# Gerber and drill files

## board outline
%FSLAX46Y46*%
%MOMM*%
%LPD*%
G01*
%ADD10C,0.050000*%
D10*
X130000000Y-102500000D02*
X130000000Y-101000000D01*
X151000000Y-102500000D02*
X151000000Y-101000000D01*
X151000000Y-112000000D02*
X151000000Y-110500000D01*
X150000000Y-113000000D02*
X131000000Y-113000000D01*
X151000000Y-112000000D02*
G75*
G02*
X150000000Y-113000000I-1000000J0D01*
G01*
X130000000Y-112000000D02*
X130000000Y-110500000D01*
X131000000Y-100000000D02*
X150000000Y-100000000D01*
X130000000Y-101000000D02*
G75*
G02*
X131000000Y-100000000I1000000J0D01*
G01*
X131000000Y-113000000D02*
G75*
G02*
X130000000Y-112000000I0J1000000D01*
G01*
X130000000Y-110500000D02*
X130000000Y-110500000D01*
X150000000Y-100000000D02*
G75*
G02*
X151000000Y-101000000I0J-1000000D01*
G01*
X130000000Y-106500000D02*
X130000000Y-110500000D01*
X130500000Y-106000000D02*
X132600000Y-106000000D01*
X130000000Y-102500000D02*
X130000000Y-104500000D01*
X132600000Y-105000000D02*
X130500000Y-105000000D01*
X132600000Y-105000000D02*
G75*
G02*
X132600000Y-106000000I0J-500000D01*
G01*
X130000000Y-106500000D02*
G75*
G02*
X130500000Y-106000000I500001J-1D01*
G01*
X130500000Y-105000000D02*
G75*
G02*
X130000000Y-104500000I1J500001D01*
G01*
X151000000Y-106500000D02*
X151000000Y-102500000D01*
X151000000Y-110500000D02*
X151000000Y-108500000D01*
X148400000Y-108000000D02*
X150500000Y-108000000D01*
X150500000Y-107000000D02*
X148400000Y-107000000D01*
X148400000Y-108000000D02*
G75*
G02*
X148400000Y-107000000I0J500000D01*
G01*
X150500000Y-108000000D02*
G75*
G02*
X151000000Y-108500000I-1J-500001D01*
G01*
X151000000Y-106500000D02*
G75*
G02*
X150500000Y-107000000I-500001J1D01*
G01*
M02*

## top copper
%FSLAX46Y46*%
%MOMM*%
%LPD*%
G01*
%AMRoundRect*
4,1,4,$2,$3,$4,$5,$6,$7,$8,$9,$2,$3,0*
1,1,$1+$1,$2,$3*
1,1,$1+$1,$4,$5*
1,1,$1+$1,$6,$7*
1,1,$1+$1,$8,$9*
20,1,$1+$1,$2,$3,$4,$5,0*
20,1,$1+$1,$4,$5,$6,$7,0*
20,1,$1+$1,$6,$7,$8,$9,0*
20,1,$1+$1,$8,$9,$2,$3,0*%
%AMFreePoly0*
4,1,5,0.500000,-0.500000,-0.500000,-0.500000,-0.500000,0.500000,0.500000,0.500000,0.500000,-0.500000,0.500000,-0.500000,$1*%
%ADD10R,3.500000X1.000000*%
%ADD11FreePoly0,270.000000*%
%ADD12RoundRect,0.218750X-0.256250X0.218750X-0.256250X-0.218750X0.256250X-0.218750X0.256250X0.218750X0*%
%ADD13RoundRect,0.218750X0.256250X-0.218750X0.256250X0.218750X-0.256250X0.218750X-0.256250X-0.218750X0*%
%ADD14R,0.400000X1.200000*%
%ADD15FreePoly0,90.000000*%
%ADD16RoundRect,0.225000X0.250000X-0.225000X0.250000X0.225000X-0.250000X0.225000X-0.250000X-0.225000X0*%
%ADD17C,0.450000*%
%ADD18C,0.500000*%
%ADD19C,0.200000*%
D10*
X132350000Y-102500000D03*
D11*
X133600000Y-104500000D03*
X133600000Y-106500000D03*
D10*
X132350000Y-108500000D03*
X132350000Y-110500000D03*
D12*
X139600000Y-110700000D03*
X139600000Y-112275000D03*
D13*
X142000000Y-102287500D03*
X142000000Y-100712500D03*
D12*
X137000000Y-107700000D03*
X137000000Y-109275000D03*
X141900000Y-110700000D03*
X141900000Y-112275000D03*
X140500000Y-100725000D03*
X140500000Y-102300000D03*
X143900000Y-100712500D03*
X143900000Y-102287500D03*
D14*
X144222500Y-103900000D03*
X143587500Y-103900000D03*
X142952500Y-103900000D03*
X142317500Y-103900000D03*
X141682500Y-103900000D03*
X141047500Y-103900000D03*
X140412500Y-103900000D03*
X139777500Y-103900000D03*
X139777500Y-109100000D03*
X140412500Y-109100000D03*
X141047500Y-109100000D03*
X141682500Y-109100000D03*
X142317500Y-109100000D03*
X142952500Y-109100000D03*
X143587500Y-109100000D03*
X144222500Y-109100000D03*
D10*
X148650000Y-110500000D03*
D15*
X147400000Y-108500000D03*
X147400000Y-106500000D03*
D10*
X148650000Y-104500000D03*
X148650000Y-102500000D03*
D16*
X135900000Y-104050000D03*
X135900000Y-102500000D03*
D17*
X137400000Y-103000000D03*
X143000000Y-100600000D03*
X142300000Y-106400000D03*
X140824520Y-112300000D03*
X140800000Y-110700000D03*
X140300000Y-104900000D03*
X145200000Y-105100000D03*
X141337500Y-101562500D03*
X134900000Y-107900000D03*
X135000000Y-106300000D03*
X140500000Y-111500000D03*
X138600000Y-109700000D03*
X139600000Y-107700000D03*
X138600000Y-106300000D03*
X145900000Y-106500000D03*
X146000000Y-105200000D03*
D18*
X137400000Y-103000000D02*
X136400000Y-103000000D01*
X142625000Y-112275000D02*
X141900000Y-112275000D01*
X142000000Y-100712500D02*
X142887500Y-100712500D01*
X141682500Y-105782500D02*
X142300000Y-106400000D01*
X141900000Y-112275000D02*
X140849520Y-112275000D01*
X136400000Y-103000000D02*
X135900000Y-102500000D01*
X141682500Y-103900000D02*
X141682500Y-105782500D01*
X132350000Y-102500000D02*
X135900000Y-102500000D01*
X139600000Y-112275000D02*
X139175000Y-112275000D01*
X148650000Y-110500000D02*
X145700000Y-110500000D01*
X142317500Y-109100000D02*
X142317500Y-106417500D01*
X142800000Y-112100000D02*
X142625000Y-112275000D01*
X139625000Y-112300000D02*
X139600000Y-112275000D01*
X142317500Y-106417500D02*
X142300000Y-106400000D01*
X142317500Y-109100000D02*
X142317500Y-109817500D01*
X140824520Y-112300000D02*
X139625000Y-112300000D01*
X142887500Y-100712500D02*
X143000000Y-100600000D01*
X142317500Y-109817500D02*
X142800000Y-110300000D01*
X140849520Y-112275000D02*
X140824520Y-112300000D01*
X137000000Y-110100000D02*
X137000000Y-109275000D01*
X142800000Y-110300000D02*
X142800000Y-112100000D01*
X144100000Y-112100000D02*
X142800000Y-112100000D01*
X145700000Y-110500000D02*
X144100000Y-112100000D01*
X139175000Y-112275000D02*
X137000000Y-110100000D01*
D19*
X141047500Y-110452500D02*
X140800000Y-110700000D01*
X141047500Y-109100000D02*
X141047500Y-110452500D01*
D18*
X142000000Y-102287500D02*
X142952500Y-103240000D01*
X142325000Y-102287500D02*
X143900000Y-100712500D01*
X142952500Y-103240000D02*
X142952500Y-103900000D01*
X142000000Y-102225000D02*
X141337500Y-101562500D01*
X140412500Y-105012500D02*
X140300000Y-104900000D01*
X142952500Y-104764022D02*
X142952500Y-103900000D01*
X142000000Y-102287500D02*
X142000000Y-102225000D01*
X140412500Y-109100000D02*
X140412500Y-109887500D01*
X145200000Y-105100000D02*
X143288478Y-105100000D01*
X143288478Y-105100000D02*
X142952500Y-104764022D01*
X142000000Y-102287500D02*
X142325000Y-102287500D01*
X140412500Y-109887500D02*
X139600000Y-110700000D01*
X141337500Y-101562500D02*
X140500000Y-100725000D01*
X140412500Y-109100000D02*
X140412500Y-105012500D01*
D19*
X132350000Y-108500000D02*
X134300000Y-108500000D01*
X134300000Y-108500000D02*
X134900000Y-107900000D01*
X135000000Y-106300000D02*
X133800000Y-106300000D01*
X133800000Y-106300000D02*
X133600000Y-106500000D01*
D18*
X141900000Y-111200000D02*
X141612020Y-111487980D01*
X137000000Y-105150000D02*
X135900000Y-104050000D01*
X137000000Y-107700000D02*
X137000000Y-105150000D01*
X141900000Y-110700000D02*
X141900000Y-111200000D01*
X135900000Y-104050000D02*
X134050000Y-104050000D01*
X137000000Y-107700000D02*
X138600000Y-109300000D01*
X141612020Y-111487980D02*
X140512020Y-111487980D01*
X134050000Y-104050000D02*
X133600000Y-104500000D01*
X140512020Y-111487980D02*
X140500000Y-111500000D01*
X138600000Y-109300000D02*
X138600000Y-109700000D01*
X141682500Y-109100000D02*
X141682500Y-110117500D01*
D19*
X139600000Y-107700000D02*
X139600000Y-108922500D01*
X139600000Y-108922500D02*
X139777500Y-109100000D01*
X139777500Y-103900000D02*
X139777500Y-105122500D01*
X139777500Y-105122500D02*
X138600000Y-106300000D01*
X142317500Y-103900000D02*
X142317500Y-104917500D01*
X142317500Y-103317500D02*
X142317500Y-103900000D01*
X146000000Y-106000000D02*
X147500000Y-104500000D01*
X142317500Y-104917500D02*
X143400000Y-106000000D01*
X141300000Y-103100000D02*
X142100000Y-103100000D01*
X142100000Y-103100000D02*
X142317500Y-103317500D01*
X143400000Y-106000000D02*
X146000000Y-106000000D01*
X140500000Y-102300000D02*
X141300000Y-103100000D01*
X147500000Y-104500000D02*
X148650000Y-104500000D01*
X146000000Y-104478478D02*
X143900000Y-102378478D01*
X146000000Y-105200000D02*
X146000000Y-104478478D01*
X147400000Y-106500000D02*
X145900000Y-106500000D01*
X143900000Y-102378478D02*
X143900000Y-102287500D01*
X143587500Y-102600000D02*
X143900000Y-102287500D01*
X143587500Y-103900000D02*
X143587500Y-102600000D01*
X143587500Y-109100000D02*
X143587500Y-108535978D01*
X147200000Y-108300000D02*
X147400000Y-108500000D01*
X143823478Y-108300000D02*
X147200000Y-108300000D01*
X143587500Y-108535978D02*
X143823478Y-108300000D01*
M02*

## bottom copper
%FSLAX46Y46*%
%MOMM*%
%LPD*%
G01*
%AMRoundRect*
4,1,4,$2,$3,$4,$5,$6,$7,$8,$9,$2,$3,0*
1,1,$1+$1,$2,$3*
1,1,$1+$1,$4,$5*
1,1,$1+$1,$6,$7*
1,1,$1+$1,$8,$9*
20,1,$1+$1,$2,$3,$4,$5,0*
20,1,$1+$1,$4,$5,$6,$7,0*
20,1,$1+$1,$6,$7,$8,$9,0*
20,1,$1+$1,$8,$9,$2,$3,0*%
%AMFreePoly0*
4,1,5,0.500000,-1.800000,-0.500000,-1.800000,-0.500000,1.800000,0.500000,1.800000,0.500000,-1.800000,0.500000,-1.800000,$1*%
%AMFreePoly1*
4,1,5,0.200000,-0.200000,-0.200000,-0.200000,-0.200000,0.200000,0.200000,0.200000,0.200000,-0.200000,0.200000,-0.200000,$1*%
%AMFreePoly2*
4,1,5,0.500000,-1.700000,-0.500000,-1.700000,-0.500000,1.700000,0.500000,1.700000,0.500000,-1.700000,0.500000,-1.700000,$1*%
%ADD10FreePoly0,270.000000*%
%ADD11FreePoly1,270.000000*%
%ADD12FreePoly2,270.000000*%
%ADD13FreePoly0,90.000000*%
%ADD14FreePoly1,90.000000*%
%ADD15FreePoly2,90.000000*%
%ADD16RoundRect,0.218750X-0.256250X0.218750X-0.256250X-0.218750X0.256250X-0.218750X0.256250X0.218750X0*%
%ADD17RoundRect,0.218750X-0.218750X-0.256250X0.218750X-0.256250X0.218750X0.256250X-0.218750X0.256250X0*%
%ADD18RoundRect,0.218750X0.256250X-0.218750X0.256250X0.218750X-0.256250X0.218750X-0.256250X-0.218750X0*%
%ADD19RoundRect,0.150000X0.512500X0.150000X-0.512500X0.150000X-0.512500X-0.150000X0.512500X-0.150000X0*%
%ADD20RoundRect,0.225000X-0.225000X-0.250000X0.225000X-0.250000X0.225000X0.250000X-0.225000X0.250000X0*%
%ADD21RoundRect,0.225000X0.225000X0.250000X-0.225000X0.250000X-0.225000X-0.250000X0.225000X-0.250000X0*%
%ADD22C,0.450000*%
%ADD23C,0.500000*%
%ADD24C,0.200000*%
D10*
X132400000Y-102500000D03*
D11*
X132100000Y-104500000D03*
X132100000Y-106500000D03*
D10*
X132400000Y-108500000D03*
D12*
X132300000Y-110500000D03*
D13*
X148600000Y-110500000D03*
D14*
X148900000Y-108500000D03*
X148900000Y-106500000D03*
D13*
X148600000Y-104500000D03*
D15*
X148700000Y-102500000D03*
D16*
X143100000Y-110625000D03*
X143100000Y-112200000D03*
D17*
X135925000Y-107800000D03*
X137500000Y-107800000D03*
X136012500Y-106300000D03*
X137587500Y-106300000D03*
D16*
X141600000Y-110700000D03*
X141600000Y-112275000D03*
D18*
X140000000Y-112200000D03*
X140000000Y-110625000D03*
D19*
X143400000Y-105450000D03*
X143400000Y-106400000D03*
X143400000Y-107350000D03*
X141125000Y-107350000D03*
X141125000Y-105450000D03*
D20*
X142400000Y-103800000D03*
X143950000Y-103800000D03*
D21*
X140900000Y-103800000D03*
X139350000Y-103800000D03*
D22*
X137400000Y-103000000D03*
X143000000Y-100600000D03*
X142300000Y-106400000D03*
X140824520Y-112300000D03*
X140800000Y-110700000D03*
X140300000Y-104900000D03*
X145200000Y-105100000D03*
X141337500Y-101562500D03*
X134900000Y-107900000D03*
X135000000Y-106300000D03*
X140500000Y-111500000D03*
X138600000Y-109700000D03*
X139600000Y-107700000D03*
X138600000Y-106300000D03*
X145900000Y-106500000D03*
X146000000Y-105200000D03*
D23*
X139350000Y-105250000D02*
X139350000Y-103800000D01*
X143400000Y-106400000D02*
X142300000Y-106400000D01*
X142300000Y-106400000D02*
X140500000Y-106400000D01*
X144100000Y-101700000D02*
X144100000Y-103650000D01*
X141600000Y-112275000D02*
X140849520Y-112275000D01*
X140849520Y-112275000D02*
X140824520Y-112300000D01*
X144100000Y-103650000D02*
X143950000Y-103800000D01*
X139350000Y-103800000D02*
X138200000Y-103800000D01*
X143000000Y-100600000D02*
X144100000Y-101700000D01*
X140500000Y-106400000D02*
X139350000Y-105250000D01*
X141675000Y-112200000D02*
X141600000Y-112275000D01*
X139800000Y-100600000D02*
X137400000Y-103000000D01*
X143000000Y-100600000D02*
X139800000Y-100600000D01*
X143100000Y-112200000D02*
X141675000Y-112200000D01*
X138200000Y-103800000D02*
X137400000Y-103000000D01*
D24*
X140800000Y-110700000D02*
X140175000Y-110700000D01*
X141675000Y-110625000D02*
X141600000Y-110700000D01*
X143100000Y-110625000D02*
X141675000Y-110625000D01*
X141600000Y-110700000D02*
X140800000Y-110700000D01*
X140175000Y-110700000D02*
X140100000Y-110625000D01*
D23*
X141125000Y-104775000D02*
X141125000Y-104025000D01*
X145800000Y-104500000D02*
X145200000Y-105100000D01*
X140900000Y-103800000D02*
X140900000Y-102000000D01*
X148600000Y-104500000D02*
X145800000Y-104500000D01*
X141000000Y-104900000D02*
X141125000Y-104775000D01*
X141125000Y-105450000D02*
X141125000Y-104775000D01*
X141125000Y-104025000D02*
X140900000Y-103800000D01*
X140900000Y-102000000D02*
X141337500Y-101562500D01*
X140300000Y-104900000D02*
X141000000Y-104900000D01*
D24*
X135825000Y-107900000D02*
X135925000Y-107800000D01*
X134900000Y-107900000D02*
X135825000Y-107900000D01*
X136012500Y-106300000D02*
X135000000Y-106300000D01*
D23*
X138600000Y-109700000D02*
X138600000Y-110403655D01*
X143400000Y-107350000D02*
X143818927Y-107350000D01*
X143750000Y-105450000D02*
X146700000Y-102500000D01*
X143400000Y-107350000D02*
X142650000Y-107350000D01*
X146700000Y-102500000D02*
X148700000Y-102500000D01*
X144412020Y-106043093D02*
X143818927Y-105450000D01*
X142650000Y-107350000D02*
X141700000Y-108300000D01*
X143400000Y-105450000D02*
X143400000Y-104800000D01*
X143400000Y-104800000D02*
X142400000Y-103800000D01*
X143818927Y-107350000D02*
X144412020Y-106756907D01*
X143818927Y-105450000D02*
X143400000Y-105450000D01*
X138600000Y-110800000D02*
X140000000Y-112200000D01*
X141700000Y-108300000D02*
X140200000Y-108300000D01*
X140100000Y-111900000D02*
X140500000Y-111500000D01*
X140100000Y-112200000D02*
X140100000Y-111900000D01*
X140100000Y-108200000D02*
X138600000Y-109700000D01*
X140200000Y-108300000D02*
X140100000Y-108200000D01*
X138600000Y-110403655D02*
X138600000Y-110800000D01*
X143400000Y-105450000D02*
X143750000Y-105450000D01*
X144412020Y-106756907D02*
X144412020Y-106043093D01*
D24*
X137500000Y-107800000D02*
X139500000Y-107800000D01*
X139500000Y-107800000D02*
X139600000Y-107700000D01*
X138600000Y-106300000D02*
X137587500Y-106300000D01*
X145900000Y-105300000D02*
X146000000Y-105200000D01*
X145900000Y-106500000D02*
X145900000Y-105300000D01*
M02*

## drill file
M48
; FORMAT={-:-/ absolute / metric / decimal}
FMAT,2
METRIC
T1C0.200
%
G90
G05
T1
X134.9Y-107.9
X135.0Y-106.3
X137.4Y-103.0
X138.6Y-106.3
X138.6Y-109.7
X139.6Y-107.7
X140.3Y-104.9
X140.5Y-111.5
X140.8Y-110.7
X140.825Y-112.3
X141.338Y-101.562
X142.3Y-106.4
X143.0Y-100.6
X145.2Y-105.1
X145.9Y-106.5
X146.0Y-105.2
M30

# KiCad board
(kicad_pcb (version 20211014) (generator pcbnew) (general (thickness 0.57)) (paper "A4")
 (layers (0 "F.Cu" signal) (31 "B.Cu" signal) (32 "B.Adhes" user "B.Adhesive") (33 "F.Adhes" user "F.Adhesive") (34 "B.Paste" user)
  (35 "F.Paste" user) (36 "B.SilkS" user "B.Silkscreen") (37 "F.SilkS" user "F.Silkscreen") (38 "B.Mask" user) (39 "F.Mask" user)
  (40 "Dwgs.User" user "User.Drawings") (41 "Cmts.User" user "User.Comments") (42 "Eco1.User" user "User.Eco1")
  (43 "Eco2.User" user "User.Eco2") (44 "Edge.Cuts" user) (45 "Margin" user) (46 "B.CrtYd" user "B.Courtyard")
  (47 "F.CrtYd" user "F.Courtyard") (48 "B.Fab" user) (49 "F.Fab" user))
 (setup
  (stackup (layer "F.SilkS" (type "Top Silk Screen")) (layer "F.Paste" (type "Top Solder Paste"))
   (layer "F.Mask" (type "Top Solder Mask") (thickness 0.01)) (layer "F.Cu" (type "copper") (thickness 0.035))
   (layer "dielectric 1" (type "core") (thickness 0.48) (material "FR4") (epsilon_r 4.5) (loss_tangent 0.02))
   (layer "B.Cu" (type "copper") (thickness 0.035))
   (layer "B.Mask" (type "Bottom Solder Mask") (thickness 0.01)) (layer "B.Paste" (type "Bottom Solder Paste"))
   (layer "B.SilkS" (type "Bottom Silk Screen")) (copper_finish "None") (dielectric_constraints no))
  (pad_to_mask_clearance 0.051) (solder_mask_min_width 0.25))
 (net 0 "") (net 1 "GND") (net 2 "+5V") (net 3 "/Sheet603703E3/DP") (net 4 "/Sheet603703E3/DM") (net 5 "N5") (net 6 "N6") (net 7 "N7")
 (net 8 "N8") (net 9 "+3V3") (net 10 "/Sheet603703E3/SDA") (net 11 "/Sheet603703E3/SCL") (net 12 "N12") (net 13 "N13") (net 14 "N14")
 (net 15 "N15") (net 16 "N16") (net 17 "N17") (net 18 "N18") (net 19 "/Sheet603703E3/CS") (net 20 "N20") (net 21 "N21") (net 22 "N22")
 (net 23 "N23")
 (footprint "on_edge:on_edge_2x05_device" (layer "F.Cu") (at 130 106.5 -90)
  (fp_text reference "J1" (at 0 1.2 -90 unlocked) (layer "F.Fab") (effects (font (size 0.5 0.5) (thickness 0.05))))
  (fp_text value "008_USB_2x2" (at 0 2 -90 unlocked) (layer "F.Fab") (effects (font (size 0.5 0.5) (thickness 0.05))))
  (fp_line (start 0 0) (end 4 0) (layer "Edge.Cuts") (width 0.05))
  (fp_line (start -0.5 -0.5) (end -0.5 -2.6) (layer "Edge.Cuts") (width 0.05))
  (fp_line (start -4 0) (end -2 0) (layer "Edge.Cuts") (width 0.05))
  (fp_line (start -1.5 -2.6) (end -1.5 -0.5) (layer "Edge.Cuts") (width 0.05))
  (fp_arc (start -1.5 -2.6) (mid -1 -3.1) (end -0.5 -2.6) (layer "Edge.Cuts") (width 0.05))
  (fp_arc (start 0 0) (mid -0.353553 -0.146447) (end -0.5 -0.5) (layer "Edge.Cuts") (width 0.05))
  (fp_arc (start -1.5 -0.5) (mid -1.646447 -0.146447) (end -2 0) (layer "Edge.Cuts") (width 0.05))
  (pad "1" smd rect locked (at -4 -2.35 90) (size 1 3.5) (layers "F.Cu" "F.Mask") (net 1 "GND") (zone_connect 0))
  (pad "2" smd custom locked (at -2 -3.6 270) (size 1 1) (layers "F.Cu" "F.Mask") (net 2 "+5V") (zone_connect 0)
   (options (clearance outline) (anchor rect)) (primitives))
  (pad "3" smd custom locked (at 0 -3.6 270) (size 1 1) (layers "F.Cu" "F.Mask") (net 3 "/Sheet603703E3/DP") (zone_connect 0)
   (options (clearance outline) (anchor rect)) (primitives))
  (pad "4" smd rect locked (at 2 -2.35 90) (size 1 3.5) (layers "F.Cu" "F.Mask") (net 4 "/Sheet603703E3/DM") (zone_connect 0))
  (pad "5" smd rect locked (at 4 -2.35 90) (size 1 3.5) (layers "F.Cu" "F.Mask") (zone_connect 0))
  (pad "6" smd custom locked (at -4 -2.4 270) (size 1 3.6) (layers "B.Cu" "B.Mask") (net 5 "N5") (zone_connect 0)
   (options (clearance outline) (anchor rect)) (primitives))
  (pad "7" smd custom locked (at -2 -2.1 270) (size 0.4 0.4) (layers "B.Cu" "B.Mask") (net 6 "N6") (zone_connect 0)
   (options (clearance outline) (anchor rect)) (primitives))
  (pad "8" smd custom locked (at 0 -2.1 270) (size 0.4 0.4) (layers "B.Cu" "B.Mask") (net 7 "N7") (zone_connect 0)
   (options (clearance outline) (anchor rect)) (primitives))
  (pad "9" smd custom locked (at 2 -2.4 270) (size 1 3.6) (layers "B.Cu" "B.Mask") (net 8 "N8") (zone_connect 0)
   (options (clearance outline) (anchor rect)) (primitives))
  (pad "10" smd custom locked (at 4 -2.3 270) (size 1 3.4) (layers "B.Cu" "B.Mask") (zone_connect 0)
   (options (clearance outline) (anchor rect)) (primitives)))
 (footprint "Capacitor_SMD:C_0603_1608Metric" (layer "F.Cu") (at 139.6 111.4875 -90)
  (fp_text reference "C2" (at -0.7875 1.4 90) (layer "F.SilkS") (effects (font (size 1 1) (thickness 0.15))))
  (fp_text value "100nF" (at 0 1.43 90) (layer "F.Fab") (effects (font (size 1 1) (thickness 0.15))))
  (pad "1" smd roundrect locked (at -0.7875 0 270) (size 0.875 0.95) (layers "F.Cu" "F.Paste" "F.Mask") (roundrect_rratio 0.25)
   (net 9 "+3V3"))
  (pad "2" smd roundrect locked (at 0.7875 0 270) (size 0.875 0.95) (layers "F.Cu" "F.Paste" "F.Mask") (roundrect_rratio 0.25) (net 1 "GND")))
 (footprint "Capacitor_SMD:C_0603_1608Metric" (layer "F.Cu") (at 142 101.5 90)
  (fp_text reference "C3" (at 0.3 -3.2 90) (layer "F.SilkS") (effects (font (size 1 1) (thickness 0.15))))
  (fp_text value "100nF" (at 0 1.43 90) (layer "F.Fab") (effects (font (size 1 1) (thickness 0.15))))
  (pad "1" smd roundrect locked (at -0.7875 0 90) (size 0.875 0.95) (layers "F.Cu" "F.Paste" "F.Mask") (roundrect_rratio 0.25)
   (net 9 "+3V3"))
  (pad "2" smd roundrect locked (at 0.7875 0 90) (size 0.875 0.95) (layers "F.Cu" "F.Paste" "F.Mask") (roundrect_rratio 0.25) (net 1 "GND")))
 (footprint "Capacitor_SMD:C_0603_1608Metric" (layer "F.Cu") (at 137 108.4875 -90)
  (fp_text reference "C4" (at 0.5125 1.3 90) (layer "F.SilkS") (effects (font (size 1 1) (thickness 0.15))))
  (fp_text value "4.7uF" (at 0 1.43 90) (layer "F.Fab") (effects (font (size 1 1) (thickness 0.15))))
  (pad "1" smd roundrect locked (at -0.7875 0 270) (size 0.875 0.95) (layers "F.Cu" "F.Paste" "F.Mask") (roundrect_rratio 0.25)
   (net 2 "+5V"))
  (pad "2" smd roundrect locked (at 0.7875 0 270) (size 0.875 0.95) (layers "F.Cu" "F.Paste" "F.Mask") (roundrect_rratio 0.25) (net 1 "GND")))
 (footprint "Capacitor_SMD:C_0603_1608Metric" (layer "F.Cu") (at 141.9 111.4875 -90)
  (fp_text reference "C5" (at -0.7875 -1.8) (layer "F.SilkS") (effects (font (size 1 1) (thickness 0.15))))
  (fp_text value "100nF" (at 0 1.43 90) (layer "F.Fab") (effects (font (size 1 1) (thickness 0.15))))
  (pad "1" smd roundrect locked (at -0.7875 0 270) (size 0.875 0.95) (layers "F.Cu" "F.Paste" "F.Mask") (roundrect_rratio 0.25)
   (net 2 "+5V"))
  (pad "2" smd roundrect locked (at 0.7875 0 270) (size 0.875 0.95) (layers "F.Cu" "F.Paste" "F.Mask") (roundrect_rratio 0.25) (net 1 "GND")))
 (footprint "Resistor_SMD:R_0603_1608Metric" (layer "F.Cu") (at 140.5 101.5125 -90)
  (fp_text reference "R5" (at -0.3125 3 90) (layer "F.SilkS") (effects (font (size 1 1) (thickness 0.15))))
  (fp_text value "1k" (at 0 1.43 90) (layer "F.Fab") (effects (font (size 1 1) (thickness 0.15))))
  (pad "1" smd roundrect locked (at -0.7875 0 270) (size 0.875 0.95) (layers "F.Cu" "F.Paste" "F.Mask") (roundrect_rratio 0.25)
   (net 9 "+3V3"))
  (pad "2" smd roundrect locked (at 0.7875 0 270) (size 0.875 0.95) (layers "F.Cu" "F.Paste" "F.Mask") (roundrect_rratio 0.25)
   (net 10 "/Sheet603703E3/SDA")))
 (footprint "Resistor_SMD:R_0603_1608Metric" (layer "F.Cu") (at 143.9 101.5 -90)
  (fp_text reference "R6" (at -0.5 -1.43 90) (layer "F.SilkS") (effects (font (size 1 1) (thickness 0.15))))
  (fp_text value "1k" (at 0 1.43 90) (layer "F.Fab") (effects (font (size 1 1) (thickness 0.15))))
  (pad "1" smd roundrect locked (at -0.7875 0 270) (size 0.875 0.95) (layers "F.Cu" "F.Paste" "F.Mask") (roundrect_rratio 0.25)
   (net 9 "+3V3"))
  (pad "2" smd roundrect locked (at 0.7875 0 270) (size 0.875 0.95) (layers "F.Cu" "F.Paste" "F.Mask") (roundrect_rratio 0.25)
   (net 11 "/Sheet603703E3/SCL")))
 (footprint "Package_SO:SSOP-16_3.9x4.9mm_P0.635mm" (layer "F.Cu") (at 142 106.5 -90)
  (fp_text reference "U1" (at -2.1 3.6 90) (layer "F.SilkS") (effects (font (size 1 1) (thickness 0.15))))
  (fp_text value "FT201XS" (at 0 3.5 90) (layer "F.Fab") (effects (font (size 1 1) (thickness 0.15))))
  (pad "1" smd rect locked (at -2.6 -2.2225 270) (size 1.2 0.4) (layers "F.Cu" "F.Paste" "F.Mask") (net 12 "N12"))
  (pad "2" smd rect locked (at -2.6 -1.5875 270) (size 1.2 0.4) (layers "F.Cu" "F.Paste" "F.Mask") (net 11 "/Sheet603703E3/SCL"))
  (pad "3" smd rect locked (at -2.6 -0.9525 270) (size 1.2 0.4) (layers "F.Cu" "F.Paste" "F.Mask") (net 9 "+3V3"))
  (pad "4" smd rect locked (at -2.6 -0.3175 270) (size 1.2 0.4) (layers "F.Cu" "F.Paste" "F.Mask") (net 10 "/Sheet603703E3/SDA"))
  (pad "5" smd rect locked (at -2.6 0.3175 270) (size 1.2 0.4) (layers "F.Cu" "F.Paste" "F.Mask") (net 1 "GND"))
  (pad "6" smd rect locked (at -2.6 0.9525 270) (size 1.2 0.4) (layers "F.Cu" "F.Paste" "F.Mask") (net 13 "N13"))
  (pad "7" smd rect locked (at -2.6 1.5875 270) (size 1.2 0.4) (layers "F.Cu" "F.Paste" "F.Mask") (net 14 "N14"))
  (pad "8" smd rect locked (at -2.6 2.2225 270) (size 1.2 0.4) (layers "F.Cu" "F.Paste" "F.Mask") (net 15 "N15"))
  (pad "9" smd rect locked (at 2.6 2.2225 270) (size 1.2 0.4) (layers "F.Cu" "F.Paste" "F.Mask") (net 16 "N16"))
  (pad "10" smd rect locked (at 2.6 1.5875 270) (size 1.2 0.4) (layers "F.Cu" "F.Paste" "F.Mask") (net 9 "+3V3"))
  (pad "11" smd rect locked (at 2.6 0.9525 270) (size 1.2 0.4) (layers "F.Cu" "F.Paste" "F.Mask") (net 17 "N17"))
  (pad "12" smd rect locked (at 2.6 0.3175 270) (size 1.2 0.4) (layers "F.Cu" "F.Paste" "F.Mask") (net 2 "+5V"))
  (pad "13" smd rect locked (at 2.6 -0.3175 270) (size 1.2 0.4) (layers "F.Cu" "F.Paste" "F.Mask") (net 1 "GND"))
  (pad "14" smd rect locked (at 2.6 -0.9525 270) (size 1.2 0.4) (layers "F.Cu" "F.Paste" "F.Mask") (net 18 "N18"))
  (pad "15" smd rect locked (at 2.6 -1.5875 270) (size 1.2 0.4) (layers "F.Cu" "F.Paste" "F.Mask") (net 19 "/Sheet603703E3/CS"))
  (pad "16" smd rect locked (at 2.6 -2.2225 270) (size 1.2 0.4) (layers "F.Cu" "F.Paste" "F.Mask") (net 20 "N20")))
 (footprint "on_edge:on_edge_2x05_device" (layer "F.Cu") (at 151 106.5 90)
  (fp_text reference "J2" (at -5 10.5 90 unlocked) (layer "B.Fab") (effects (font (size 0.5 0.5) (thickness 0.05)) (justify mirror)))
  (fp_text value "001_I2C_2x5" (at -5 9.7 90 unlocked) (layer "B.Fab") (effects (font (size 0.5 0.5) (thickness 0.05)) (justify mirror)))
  (fp_line (start 0 0) (end 4 0) (layer "Edge.Cuts") (width 0.05))
  (fp_line (start -4 0) (end -2 0) (layer "Edge.Cuts") (width 0.05))
  (fp_line (start -1.5 -2.6) (end -1.5 -0.5) (layer "Edge.Cuts") (width 0.05))
  (fp_line (start -0.5 -0.5) (end -0.5 -2.6) (layer "Edge.Cuts") (width 0.05))
  (fp_arc (start -1.5 -2.6) (mid -1 -3.1) (end -0.5 -2.6) (layer "Edge.Cuts") (width 0.05))
  (fp_arc (start -1.5 -0.5) (mid -1.646447 -0.146447) (end -2 0) (layer "Edge.Cuts") (width 0.05))
  (fp_arc (start 0 0) (mid -0.353553 -0.146447) (end -0.5 -0.5) (layer "Edge.Cuts") (width 0.05))
  (pad "1" smd rect locked (at -4 -2.35 270) (size 1 3.5) (layers "F.Cu" "F.Mask") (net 1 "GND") (zone_connect 0))
  (pad "2" smd custom locked (at -2 -3.6 90) (size 1 1) (layers "F.Cu" "F.Mask") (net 19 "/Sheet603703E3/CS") (zone_connect 0)
   (options (clearance outline) (anchor rect)) (primitives))
  (pad "3" smd custom locked (at 0 -3.6 90) (size 1 1) (layers "F.Cu" "F.Mask") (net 11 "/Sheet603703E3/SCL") (zone_connect 0)
   (options (clearance outline) (anchor rect)) (primitives))
  (pad "4" smd rect locked (at 2 -2.35 270) (size 1 3.5) (layers "F.Cu" "F.Mask") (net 10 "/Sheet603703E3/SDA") (zone_connect 0))
  (pad "5" smd rect locked (at 4 -2.35 270) (size 1 3.5) (layers "F.Cu" "F.Mask") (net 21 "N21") (zone_connect 0))
  (pad "6" smd custom locked (at -4 -2.4 90) (size 1 3.6) (layers "B.Cu" "B.Mask") (zone_connect 0)
   (options (clearance outline) (anchor rect)) (primitives))
  (pad "7" smd custom locked (at -2 -2.1 90) (size 0.4 0.4) (layers "B.Cu" "B.Mask") (zone_connect 0)
   (options (clearance outline) (anchor rect)) (primitives))
  (pad "8" smd custom locked (at 0 -2.1 90) (size 0.4 0.4) (layers "B.Cu" "B.Mask") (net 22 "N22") (zone_connect 0)
   (options (clearance outline) (anchor rect)) (primitives))
  (pad "9" smd custom locked (at 2 -2.4 90) (size 1 3.6) (layers "B.Cu" "B.Mask") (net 9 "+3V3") (zone_connect 0)
   (options (clearance outline) (anchor rect)) (primitives))
  (pad "10" smd custom locked (at 4 -2.3 90) (size 1 3.4) (layers "B.Cu" "B.Mask") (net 2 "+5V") (zone_connect 0)
   (options (clearance outline) (anchor rect)) (primitives)))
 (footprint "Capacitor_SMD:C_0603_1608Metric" (layer "F.Cu") (at 135.9 103.275 90)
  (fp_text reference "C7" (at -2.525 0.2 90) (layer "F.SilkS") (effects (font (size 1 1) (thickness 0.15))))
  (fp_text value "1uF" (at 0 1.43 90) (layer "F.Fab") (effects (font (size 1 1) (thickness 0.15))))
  (pad "1" smd roundrect locked (at -0.775 0 90) (size 0.9 0.95) (layers "F.Cu" "F.Paste" "F.Mask") (roundrect_rratio 0.25) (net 2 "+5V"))
  (pad "2" smd roundrect locked (at 0.775 0 90) (size 0.9 0.95) (layers "F.Cu" "F.Paste" "F.Mask") (roundrect_rratio 0.25) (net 1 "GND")))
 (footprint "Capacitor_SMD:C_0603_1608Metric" (layer "B.Cu") (at 143.1 111.4125 -90)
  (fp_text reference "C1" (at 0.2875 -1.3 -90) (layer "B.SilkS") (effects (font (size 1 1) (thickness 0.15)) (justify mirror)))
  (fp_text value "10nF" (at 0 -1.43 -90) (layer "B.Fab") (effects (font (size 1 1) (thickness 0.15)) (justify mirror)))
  (pad "1" smd roundrect locked (at -0.7875 0 270) (size 0.875 0.95) (layers "B.Cu" "B.Paste" "B.Mask") (roundrect_rratio 0.25)
   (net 17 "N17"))
  (pad "2" smd roundrect locked (at 0.7875 0 270) (size 0.875 0.95) (layers "B.Cu" "B.Paste" "B.Mask") (roundrect_rratio 0.25) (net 1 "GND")))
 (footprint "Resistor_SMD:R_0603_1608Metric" (layer "B.Cu") (at 136.7125 107.8)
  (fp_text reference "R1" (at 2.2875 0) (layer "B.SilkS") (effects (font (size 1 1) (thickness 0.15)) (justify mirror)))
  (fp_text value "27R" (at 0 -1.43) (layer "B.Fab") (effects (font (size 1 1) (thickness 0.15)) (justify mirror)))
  (pad "1" smd roundrect locked (at -0.7875 0) (size 0.875 0.95) (layers "B.Cu" "B.Paste" "B.Mask") (roundrect_rratio 0.25)
   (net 4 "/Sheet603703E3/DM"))
  (pad "2" smd roundrect locked (at 0.7875 0) (size 0.875 0.95) (layers "B.Cu" "B.Paste" "B.Mask") (roundrect_rratio 0.25) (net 16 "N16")))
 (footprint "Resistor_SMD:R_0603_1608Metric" (layer "B.Cu") (at 136.8 106.3)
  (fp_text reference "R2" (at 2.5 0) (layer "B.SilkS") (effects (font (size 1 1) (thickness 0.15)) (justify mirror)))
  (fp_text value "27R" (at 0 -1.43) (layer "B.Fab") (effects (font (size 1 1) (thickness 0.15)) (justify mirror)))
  (pad "1" smd roundrect locked (at -0.7875 0) (size 0.875 0.95) (layers "B.Cu" "B.Paste" "B.Mask") (roundrect_rratio 0.25)
   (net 3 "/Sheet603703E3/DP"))
  (pad "2" smd roundrect locked (at 0.7875 0) (size 0.875 0.95) (layers "B.Cu" "B.Paste" "B.Mask") (roundrect_rratio 0.25) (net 15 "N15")))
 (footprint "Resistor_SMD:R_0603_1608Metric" (layer "B.Cu") (at 141.6 111.4875 -90)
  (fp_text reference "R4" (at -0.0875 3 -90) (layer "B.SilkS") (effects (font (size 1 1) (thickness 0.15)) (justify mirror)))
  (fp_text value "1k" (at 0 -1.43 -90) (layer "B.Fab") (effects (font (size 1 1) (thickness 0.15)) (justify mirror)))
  (pad "1" smd roundrect locked (at -0.7875 0 270) (size 0.875 0.95) (layers "B.Cu" "B.Paste" "B.Mask") (roundrect_rratio 0.25)
   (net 17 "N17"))
  (pad "2" smd roundrect locked (at 0.7875 0 270) (size 0.875 0.95) (layers "B.Cu" "B.Paste" "B.Mask") (roundrect_rratio 0.25) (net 1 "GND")))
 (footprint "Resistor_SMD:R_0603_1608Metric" (layer "B.Cu") (at 140 111.4125 90)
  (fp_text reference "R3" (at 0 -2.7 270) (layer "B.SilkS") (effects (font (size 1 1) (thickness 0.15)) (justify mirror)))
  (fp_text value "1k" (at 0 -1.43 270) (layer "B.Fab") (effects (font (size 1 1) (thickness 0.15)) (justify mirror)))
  (pad "1" smd roundrect locked (at -0.7875 0 90) (size 0.875 0.95) (layers "B.Cu" "B.Paste" "B.Mask") (roundrect_rratio 0.25) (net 2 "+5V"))
  (pad "2" smd roundrect locked (at 0.7875 0 90) (size 0.875 0.95) (layers "B.Cu" "B.Paste" "B.Mask") (roundrect_rratio 0.25) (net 17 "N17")))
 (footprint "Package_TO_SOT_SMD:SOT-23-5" (layer "B.Cu") (at 142.2625 106.4 180)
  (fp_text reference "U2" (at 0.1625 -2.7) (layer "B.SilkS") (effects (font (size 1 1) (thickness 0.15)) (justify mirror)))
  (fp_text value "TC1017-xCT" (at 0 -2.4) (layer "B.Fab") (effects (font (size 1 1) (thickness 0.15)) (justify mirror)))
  (pad "1" smd roundrect locked (at -1.1375 0.95 180) (size 1.325 0.6) (layers "B.Cu" "B.Paste" "B.Mask") (roundrect_rratio 0.25)
   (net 2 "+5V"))
  (pad "2" smd roundrect locked (at -1.1375 0 180) (size 1.325 0.6) (layers "B.Cu" "B.Paste" "B.Mask") (roundrect_rratio 0.25) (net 1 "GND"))
  (pad "3" smd roundrect locked (at -1.1375 -0.95 180) (size 1.325 0.6) (layers "B.Cu" "B.Paste" "B.Mask") (roundrect_rratio 0.25)
   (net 2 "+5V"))
  (pad "4" smd roundrect locked (at 1.1375 -0.95 180) (size 1.325 0.6) (layers "B.Cu" "B.Paste" "B.Mask") (roundrect_rratio 0.25)
   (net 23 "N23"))
  (pad "5" smd roundrect locked (at 1.1375 0.95 180) (size 1.325 0.6) (layers "B.Cu" "B.Paste" "B.Mask") (roundrect_rratio 0.25)
   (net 9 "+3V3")))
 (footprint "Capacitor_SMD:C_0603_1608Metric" (layer "B.Cu") (at 143.175 103.8)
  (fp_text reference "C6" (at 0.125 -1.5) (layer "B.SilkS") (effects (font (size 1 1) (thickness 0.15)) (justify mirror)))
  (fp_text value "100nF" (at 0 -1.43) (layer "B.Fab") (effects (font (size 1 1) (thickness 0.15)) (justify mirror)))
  (pad "1" smd roundrect locked (at -0.775 0) (size 0.9 0.95) (layers "B.Cu" "B.Paste" "B.Mask") (roundrect_rratio 0.25) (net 2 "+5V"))
  (pad "2" smd roundrect locked (at 0.775 0) (size 0.9 0.95) (layers "B.Cu" "B.Paste" "B.Mask") (roundrect_rratio 0.25) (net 1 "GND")))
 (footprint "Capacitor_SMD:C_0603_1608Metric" (layer "B.Cu") (at 140.125 103.8 180)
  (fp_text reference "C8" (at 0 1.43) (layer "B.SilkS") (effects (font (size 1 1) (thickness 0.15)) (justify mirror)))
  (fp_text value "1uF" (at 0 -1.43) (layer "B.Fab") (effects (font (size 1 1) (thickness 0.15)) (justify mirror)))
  (pad "1" smd roundrect locked (at -0.775 0 180) (size 0.9 0.95) (layers "B.Cu" "B.Paste" "B.Mask") (roundrect_rratio 0.25) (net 9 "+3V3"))
  (pad "2" smd roundrect locked (at 0.775 0 180) (size 0.9 0.95) (layers "B.Cu" "B.Paste" "B.Mask") (roundrect_rratio 0.25) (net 1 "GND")))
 (gr_line (start 130 102.5) (end 130 101) (layer "Edge.Cuts") (width 0.05))
 (gr_line (start 151 102.5) (end 151 101) (layer "Edge.Cuts") (width 0.05))
 (gr_line (start 151 112) (end 151 110.5) (layer "Edge.Cuts") (width 0.05))
 (gr_line (start 150 113) (end 131 113) (layer "Edge.Cuts") (width 0.05))
 (gr_arc (start 151 112) (mid 150.707107 112.707107) (end 150 113) (layer "Edge.Cuts") (width 0.05))
 (gr_line (start 130 112) (end 130 110.5) (layer "Edge.Cuts") (width 0.05))
 (gr_line (start 131 100) (end 150 100) (layer "Edge.Cuts") (width 0.05))
 (gr_arc (start 130 101) (mid 130.292893 100.292893) (end 131 100) (layer "Edge.Cuts") (width 0.05))
 (gr_arc (start 131 113) (mid 130.292893 112.707107) (end 130 112) (layer "Edge.Cuts") (width 0.05))
 (gr_line (start 130 110.5) (end 130 110.5) (layer "Edge.Cuts") (width 0.05))
 (gr_arc (start 150 100) (mid 150.707107 100.292893) (end 151 101) (layer "Edge.Cuts") (width 0.05))
 (segment (start 137.4 103) (end 136.4 103) (width 0.5) (layer "F.Cu") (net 1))
 (segment (start 142.625 112.275) (end 141.9 112.275) (width 0.5) (layer "F.Cu") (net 1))
 (segment (start 142 100.7125) (end 142.8875 100.7125) (width 0.5) (layer "F.Cu") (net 1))
 (segment (start 141.6825 105.7825) (end 142.3 106.4) (width 0.5) (layer "F.Cu") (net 1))
 (segment (start 141.9 112.275) (end 140.84952 112.275) (width 0.5) (layer "F.Cu") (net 1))
 (segment (start 136.4 103) (end 135.9 102.5) (width 0.5) (layer "F.Cu") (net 1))
 (segment (start 141.6825 103.9) (end 141.6825 105.7825) (width 0.5) (layer "F.Cu") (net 1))
 (segment (start 132.35 102.5) (end 135.9 102.5) (width 0.5) (layer "F.Cu") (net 1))
 (segment (start 139.6 112.275) (end 139.175 112.275) (width 0.5) (layer "F.Cu") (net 1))
 (segment (start 148.65 110.5) (end 145.7 110.5) (width 0.5) (layer "F.Cu") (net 1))
 (segment (start 142.3175 109.1) (end 142.3175 106.4175) (width 0.5) (layer "F.Cu") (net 1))
 (segment (start 142.8 112.1) (end 142.625 112.275) (width 0.5) (layer "F.Cu") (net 1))
 (segment (start 139.625 112.3) (end 139.6 112.275) (width 0.5) (layer "F.Cu") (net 1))
 (segment (start 142.3175 106.4175) (end 142.3 106.4) (width 0.5) (layer "F.Cu") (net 1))
 (segment (start 142.3175 109.1) (end 142.3175 109.8175) (width 0.5) (layer "F.Cu") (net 1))
 (segment (start 140.82452 112.3) (end 139.625 112.3) (width 0.5) (layer "F.Cu") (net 1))
 (segment (start 142.8875 100.7125) (end 143 100.6) (width 0.5) (layer "F.Cu") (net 1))
 (segment (start 142.3175 109.8175) (end 142.8 110.3) (width 0.5) (layer "F.Cu") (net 1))
 (segment (start 140.84952 112.275) (end 140.82452 112.3) (width 0.5) (layer "F.Cu") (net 1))
 (segment (start 137 110.1) (end 137 109.275) (width 0.5) (layer "F.Cu") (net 1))
 (segment (start 142.8 110.3) (end 142.8 112.1) (width 0.5) (layer "F.Cu") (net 1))
 (segment (start 144.1 112.1) (end 142.8 112.1) (width 0.5) (layer "F.Cu") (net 1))
 (segment (start 145.7 110.5) (end 144.1 112.1) (width 0.5) (layer "F.Cu") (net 1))
 (segment (start 139.175 112.275) (end 137 110.1) (width 0.5) (layer "F.Cu") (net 1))
 (via (at 137.4 103) (size 0.45) (drill 0.2) (layers "F.Cu" "B.Cu") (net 1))
 (via (at 143 100.6) (size 0.45) (drill 0.2) (layers "F.Cu" "B.Cu") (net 1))
 (via (at 142.3 106.4) (size 0.45) (drill 0.2) (layers "F.Cu" "B.Cu") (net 1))
 (via (at 140.82452 112.3) (size 0.45) (drill 0.2) (layers "F.Cu" "B.Cu") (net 1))
 (segment (start 139.35 105.25) (end 139.35 103.8) (width 0.5) (layer "B.Cu") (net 1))
 (segment (start 143.4 106.4) (end 142.3 106.4) (width 0.5) (layer "B.Cu") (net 1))
 (segment (start 142.3 106.4) (end 140.5 106.4) (width 0.5) (layer "B.Cu") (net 1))
 (segment (start 144.1 101.7) (end 144.1 103.65) (width 0.5) (layer "B.Cu") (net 1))
 (segment (start 141.6 112.275) (end 140.84952 112.275) (width 0.5) (layer "B.Cu") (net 1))
 (segment (start 140.84952 112.275) (end 140.82452 112.3) (width 0.5) (layer "B.Cu") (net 1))
 (segment (start 144.1 103.65) (end 143.95 103.8) (width 0.5) (layer "B.Cu") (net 1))
 (segment (start 139.35 103.8) (end 138.2 103.8) (width 0.5) (layer "B.Cu") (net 1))
 (segment (start 143 100.6) (end 144.1 101.7) (width 0.5) (layer "B.Cu") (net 1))
 (segment (start 140.5 106.4) (end 139.35 105.25) (width 0.5) (layer "B.Cu") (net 1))
 (segment (start 141.675 112.2) (end 141.6 112.275) (width 0.5) (layer "B.Cu") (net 1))
 (segment (start 139.8 100.6) (end 137.4 103) (width 0.5) (layer "B.Cu") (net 1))
 (segment (start 143 100.6) (end 139.8 100.6) (width 0.5) (layer "B.Cu") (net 1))
 (segment (start 143.1 112.2) (end 141.675 112.2) (width 0.5) (layer "B.Cu") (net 1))
 (segment (start 138.2 103.8) (end 137.4 103) (width 0.5) (layer "B.Cu") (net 1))
 (segment (start 141.0475 110.4525) (end 140.8 110.7) (width 0.2) (layer "F.Cu") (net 17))
 (segment (start 141.0475 109.1) (end 141.0475 110.4525) (width 0.2) (layer "F.Cu") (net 17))
 (via (at 140.8 110.7) (size 0.45) (drill 0.2) (layers "F.Cu" "B.Cu") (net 17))
 (segment (start 140.8 110.7) (end 140.175 110.7) (width 0.2) (layer "B.Cu") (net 17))
 (segment (start 141.675 110.625) (end 141.6 110.7) (width 0.2) (layer "B.Cu") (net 17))
 (segment (start 143.1 110.625) (end 141.675 110.625) (width 0.2) (layer "B.Cu") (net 17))
 (segment (start 141.6 110.7) (end 140.8 110.7) (width 0.2) (layer "B.Cu") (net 17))
 (segment (start 140.175 110.7) (end 140.1 110.625) (width 0.2) (layer "B.Cu") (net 17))
 (segment (start 142 102.2875) (end 142.9525 103.24) (width 0.5) (layer "F.Cu") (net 9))
 (segment (start 142.325 102.2875) (end 143.9 100.7125) (width 0.5) (layer "F.Cu") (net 9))
 (segment (start 142.9525 103.24) (end 142.9525 103.9) (width 0.5) (layer "F.Cu") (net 9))
 (segment (start 142 102.225) (end 141.3375 101.5625) (width 0.5) (layer "F.Cu") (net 9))
 (segment (start 140.4125 105.0125) (end 140.3 104.9) (width 0.5) (layer "F.Cu") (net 9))
 (segment (start 142.9525 104.764022) (end 142.9525 103.9) (width 0.5) (layer "F.Cu") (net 9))
 (segment (start 142 102.2875) (end 142 102.225) (width 0.5) (layer "F.Cu") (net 9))
 (segment (start 140.4125 109.1) (end 140.4125 109.8875) (width 0.5) (layer "F.Cu") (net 9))
 (segment (start 145.2 105.1) (end 143.288478 105.1) (width 0.5) (layer "F.Cu") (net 9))
 (segment (start 143.288478 105.1) (end 142.9525 104.764022) (width 0.5) (layer "F.Cu") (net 9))
 (segment (start 142 102.2875) (end 142.325 102.2875) (width 0.5) (layer "F.Cu") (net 9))
 (segment (start 140.4125 109.8875) (end 139.6 110.7) (width 0.5) (layer "F.Cu") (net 9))
 (segment (start 141.3375 101.5625) (end 140.5 100.725) (width 0.5) (layer "F.Cu") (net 9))
 (segment (start 140.4125 109.1) (end 140.4125 105.0125) (width 0.5) (layer "F.Cu") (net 9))
 (via (at 140.3 104.9) (size 0.45) (drill 0.2) (layers "F.Cu" "B.Cu") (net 9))
 (via (at 145.2 105.1) (size 0.45) (drill 0.2) (layers "F.Cu" "B.Cu") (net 9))
 (via (at 141.3375 101.5625) (size 0.45) (drill 0.2) (layers "F.Cu" "B.Cu") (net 9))
 (segment (start 141.125 104.775) (end 141.125 104.025) (width 0.5) (layer "B.Cu") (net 9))
 (segment (start 145.8 104.5) (end 145.2 105.1) (width 0.5) (layer "B.Cu") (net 9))
 (segment (start 140.9 103.8) (end 140.9 102) (width 0.5) (layer "B.Cu") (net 9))
 (segment (start 148.6 104.5) (end 145.8 104.5) (width 0.5) (layer "B.Cu") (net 9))
 (segment (start 141 104.9) (end 141.125 104.775) (width 0.5) (layer "B.Cu") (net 9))
 (segment (start 141.125 105.45) (end 141.125 104.775) (width 0.5) (layer "B.Cu") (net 9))
 (segment (start 141.125 104.025) (end 140.9 103.8) (width 0.5) (layer "B.Cu") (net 9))
 (segment (start 140.9 102) (end 141.3375 101.5625) (width 0.5) (layer "B.Cu") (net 9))
 (segment (start 140.3 104.9) (end 141 104.9) (width 0.5) (layer "B.Cu") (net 9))
 (segment (start 132.35 108.5) (end 134.3 108.5) (width 0.2) (layer "F.Cu") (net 4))
 (segment (start 134.3 108.5) (end 134.9 107.9) (width 0.2) (layer "F.Cu") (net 4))
 (via (at 134.9 107.9) (size 0.45) (drill 0.2) (layers "F.Cu" "B.Cu") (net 4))
 (segment (start 135.825 107.9) (end 135.925 107.8) (width 0.2) (layer "B.Cu") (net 4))
 (segment (start 134.9 107.9) (end 135.825 107.9) (width 0.2) (layer "B.Cu") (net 4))
 (segment (start 135 106.3) (end 133.8 106.3) (width 0.2) (layer "F.Cu") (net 3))
 (segment (start 133.8 106.3) (end 133.6 106.5) (width 0.2) (layer "F.Cu") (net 3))
 (via (at 135 106.3) (size 0.45) (drill 0.2) (layers "F.Cu" "B.Cu") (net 3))
 (segment (start 136.0125 106.3) (end 135 106.3) (width 0.2) (layer "B.Cu") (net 3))
 (segment (start 141.9 111.2) (end 141.61202 111.48798) (width 0.5) (layer "F.Cu") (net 2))
 (segment (start 137 105.15) (end 135.9 104.05) (width 0.5) (layer "F.Cu") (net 2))
 (segment (start 137 107.7) (end 137 105.15) (width 0.5) (layer "F.Cu") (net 2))
 (segment (start 141.9 110.7) (end 141.9 111.2) (width 0.5) (layer "F.Cu") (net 2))
 (segment (start 135.9 104.05) (end 134.05 104.05) (width 0.5) (layer "F.Cu") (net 2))
 (segment (start 137 107.7) (end 138.6 109.3) (width 0.5) (layer "F.Cu") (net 2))
 (segment (start 141.61202 111.48798) (end 140.51202 111.48798) (width 0.5) (layer "F.Cu") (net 2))
 (segment (start 134.05 104.05) (end 133.6 104.5) (width 0.5) (layer "F.Cu") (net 2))
 (segment (start 140.51202 111.48798) (end 140.5 111.5) (width 0.5) (layer "F.Cu") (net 2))
 (segment (start 138.6 109.3) (end 138.6 109.7) (width 0.5) (layer "F.Cu") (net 2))
 (segment (start 141.6825 109.1) (end 141.6825 110.1175) (width 0.5) (layer "F.Cu") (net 2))
 (via (at 140.5 111.5) (size 0.45) (drill 0.2) (layers "F.Cu" "B.Cu") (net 2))
 (via (at 138.6 109.7) (size 0.45) (drill 0.2) (layers "F.Cu" "B.Cu") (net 2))
 (segment (start 138.6 109.7) (end 138.6 110.403655) (width 0.5) (layer "B.Cu") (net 2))
 (segment (start 143.4 107.35) (end 143.818927 107.35) (width 0.5) (layer "B.Cu") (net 2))
 (segment (start 143.75 105.45) (end 146.7 102.5) (width 0.5) (layer "B.Cu") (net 2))
 (segment (start 143.4 107.35) (end 142.65 107.35) (width 0.5) (layer "B.Cu") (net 2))
 (segment (start 146.7 102.5) (end 148.7 102.5) (width 0.5) (layer "B.Cu") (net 2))
 (segment (start 144.41202 106.043093) (end 143.818927 105.45) (width 0.5) (layer "B.Cu") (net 2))
 (segment (start 142.65 107.35) (end 141.7 108.3) (width 0.5) (layer "B.Cu") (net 2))
 (segment (start 143.4 105.45) (end 143.4 104.8) (width 0.5) (layer "B.Cu") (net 2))
 (segment (start 143.4 104.8) (end 142.4 103.8) (width 0.5) (layer "B.Cu") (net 2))
 (segment (start 143.818927 107.35) (end 144.41202 106.756907) (width 0.5) (layer "B.Cu") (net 2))
 (segment (start 143.818927 105.45) (end 143.4 105.45) (width 0.5) (layer "B.Cu") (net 2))
 (segment (start 138.6 110.8) (end 140 112.2) (width 0.5) (layer "B.Cu") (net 2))
 (segment (start 141.7 108.3) (end 140.2 108.3) (width 0.5) (layer "B.Cu") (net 2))
 (segment (start 140.1 111.9) (end 140.5 111.5) (width 0.5) (layer "B.Cu") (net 2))
 (segment (start 140.1 112.2) (end 140.1 111.9) (width 0.5) (layer "B.Cu") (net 2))
 (segment (start 140.1 108.2) (end 138.6 109.7) (width 0.5) (layer "B.Cu") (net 2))
 (segment (start 140.2 108.3) (end 140.1 108.2) (width 0.5) (layer "B.Cu") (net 2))
 (segment (start 138.6 110.403655) (end 138.6 110.8) (width 0.5) (layer "B.Cu") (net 2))
 (segment (start 143.4 105.45) (end 143.75 105.45) (width 0.5) (layer "B.Cu") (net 2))
 (segment (start 144.41202 106.756907) (end 144.41202 106.043093) (width 0.5) (layer "B.Cu") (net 2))
 (segment (start 139.6 107.7) (end 139.6 108.9225) (width 0.2) (layer "F.Cu") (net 16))
 (segment (start 139.6 108.9225) (end 139.7775 109.1) (width 0.2) (layer "F.Cu") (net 16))
 (via (at 139.6 107.7) (size 0.45) (drill 0.2) (layers "F.Cu" "B.Cu") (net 16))
 (segment (start 137.5 107.8) (end 139.5 107.8) (width 0.2) (layer "B.Cu") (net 16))
 (segment (start 139.5 107.8) (end 139.6 107.7) (width 0.2) (layer "B.Cu") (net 16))
 (segment (start 139.7775 103.9) (end 139.7775 105.1225) (width 0.2) (layer "F.Cu") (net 15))
 (segment (start 139.7775 105.1225) (end 138.6 106.3) (width 0.2) (layer "F.Cu") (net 15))
 (via (at 138.6 106.3) (size 0.45) (drill 0.2) (layers "F.Cu" "B.Cu") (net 15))
 (segment (start 138.6 106.3) (end 137.5875 106.3) (width 0.2) (layer "B.Cu") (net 15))
 (segment (start 142.3175 103.9) (end 142.3175 104.9175) (width 0.2) (layer "F.Cu") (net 10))
 (segment (start 142.3175 103.3175) (end 142.3175 103.9) (width 0.2) (layer "F.Cu") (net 10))
 (segment (start 146 106) (end 147.5 104.5) (width 0.2) (layer "F.Cu") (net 10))
 (segment (start 142.3175 104.9175) (end 143.4 106) (width 0.2) (layer "F.Cu") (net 10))
 (segment (start 141.3 103.1) (end 142.1 103.1) (width 0.2) (layer "F.Cu") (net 10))
 (segment (start 142.1 103.1) (end 142.3175 103.3175) (width 0.2) (layer "F.Cu") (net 10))
 (segment (start 143.4 106) (end 146 106) (width 0.2) (layer "F.Cu") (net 10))
 (segment (start 140.5 102.3) (end 141.3 103.1) (width 0.2) (layer "F.Cu") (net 10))
 (segment (start 147.5 104.5) (end 148.65 104.5) (width 0.2) (layer "F.Cu") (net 10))
 (segment (start 146 104.478478) (end 143.9 102.378478) (width 0.2) (layer "F.Cu") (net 11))
 (segment (start 146 105.2) (end 146 104.478478) (width 0.2) (layer "F.Cu") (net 11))
 (segment (start 147.4 106.5) (end 145.9 106.5) (width 0.2) (layer "F.Cu") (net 11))
 (segment (start 143.9 102.378478) (end 143.9 102.2875) (width 0.2) (layer "F.Cu") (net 11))
 (segment (start 143.5875 102.6) (end 143.9 102.2875) (width 0.2) (layer "F.Cu") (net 11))
 (segment (start 143.5875 103.9) (end 143.5875 102.6) (width 0.2) (layer "F.Cu") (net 11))
 (via (at 145.9 106.5) (size 0.45) (drill 0.2) (layers "F.Cu" "B.Cu") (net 11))
 (via (at 146 105.2) (size 0.45) (drill 0.2) (layers "F.Cu" "B.Cu") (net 11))
 (segment (start 145.9 105.3) (end 146 105.2) (width 0.2) (layer "B.Cu") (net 11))
 (segment (start 145.9 106.5) (end 145.9 105.3) (width 0.2) (layer "B.Cu") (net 11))
 (segment (start 143.5875 109.1) (end 143.5875 108.535978) (width 0.2) (layer "F.Cu") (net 19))
 (segment (start 147.2 108.3) (end 147.4 108.5) (width 0.2) (layer "F.Cu") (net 19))
 (segment (start 143.823478 108.3) (end 147.2 108.3) (width 0.2) (layer "F.Cu") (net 19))
 (segment (start 143.5875 108.535978) (end 143.823478 108.3) (width 0.2) (layer "F.Cu") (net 19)))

